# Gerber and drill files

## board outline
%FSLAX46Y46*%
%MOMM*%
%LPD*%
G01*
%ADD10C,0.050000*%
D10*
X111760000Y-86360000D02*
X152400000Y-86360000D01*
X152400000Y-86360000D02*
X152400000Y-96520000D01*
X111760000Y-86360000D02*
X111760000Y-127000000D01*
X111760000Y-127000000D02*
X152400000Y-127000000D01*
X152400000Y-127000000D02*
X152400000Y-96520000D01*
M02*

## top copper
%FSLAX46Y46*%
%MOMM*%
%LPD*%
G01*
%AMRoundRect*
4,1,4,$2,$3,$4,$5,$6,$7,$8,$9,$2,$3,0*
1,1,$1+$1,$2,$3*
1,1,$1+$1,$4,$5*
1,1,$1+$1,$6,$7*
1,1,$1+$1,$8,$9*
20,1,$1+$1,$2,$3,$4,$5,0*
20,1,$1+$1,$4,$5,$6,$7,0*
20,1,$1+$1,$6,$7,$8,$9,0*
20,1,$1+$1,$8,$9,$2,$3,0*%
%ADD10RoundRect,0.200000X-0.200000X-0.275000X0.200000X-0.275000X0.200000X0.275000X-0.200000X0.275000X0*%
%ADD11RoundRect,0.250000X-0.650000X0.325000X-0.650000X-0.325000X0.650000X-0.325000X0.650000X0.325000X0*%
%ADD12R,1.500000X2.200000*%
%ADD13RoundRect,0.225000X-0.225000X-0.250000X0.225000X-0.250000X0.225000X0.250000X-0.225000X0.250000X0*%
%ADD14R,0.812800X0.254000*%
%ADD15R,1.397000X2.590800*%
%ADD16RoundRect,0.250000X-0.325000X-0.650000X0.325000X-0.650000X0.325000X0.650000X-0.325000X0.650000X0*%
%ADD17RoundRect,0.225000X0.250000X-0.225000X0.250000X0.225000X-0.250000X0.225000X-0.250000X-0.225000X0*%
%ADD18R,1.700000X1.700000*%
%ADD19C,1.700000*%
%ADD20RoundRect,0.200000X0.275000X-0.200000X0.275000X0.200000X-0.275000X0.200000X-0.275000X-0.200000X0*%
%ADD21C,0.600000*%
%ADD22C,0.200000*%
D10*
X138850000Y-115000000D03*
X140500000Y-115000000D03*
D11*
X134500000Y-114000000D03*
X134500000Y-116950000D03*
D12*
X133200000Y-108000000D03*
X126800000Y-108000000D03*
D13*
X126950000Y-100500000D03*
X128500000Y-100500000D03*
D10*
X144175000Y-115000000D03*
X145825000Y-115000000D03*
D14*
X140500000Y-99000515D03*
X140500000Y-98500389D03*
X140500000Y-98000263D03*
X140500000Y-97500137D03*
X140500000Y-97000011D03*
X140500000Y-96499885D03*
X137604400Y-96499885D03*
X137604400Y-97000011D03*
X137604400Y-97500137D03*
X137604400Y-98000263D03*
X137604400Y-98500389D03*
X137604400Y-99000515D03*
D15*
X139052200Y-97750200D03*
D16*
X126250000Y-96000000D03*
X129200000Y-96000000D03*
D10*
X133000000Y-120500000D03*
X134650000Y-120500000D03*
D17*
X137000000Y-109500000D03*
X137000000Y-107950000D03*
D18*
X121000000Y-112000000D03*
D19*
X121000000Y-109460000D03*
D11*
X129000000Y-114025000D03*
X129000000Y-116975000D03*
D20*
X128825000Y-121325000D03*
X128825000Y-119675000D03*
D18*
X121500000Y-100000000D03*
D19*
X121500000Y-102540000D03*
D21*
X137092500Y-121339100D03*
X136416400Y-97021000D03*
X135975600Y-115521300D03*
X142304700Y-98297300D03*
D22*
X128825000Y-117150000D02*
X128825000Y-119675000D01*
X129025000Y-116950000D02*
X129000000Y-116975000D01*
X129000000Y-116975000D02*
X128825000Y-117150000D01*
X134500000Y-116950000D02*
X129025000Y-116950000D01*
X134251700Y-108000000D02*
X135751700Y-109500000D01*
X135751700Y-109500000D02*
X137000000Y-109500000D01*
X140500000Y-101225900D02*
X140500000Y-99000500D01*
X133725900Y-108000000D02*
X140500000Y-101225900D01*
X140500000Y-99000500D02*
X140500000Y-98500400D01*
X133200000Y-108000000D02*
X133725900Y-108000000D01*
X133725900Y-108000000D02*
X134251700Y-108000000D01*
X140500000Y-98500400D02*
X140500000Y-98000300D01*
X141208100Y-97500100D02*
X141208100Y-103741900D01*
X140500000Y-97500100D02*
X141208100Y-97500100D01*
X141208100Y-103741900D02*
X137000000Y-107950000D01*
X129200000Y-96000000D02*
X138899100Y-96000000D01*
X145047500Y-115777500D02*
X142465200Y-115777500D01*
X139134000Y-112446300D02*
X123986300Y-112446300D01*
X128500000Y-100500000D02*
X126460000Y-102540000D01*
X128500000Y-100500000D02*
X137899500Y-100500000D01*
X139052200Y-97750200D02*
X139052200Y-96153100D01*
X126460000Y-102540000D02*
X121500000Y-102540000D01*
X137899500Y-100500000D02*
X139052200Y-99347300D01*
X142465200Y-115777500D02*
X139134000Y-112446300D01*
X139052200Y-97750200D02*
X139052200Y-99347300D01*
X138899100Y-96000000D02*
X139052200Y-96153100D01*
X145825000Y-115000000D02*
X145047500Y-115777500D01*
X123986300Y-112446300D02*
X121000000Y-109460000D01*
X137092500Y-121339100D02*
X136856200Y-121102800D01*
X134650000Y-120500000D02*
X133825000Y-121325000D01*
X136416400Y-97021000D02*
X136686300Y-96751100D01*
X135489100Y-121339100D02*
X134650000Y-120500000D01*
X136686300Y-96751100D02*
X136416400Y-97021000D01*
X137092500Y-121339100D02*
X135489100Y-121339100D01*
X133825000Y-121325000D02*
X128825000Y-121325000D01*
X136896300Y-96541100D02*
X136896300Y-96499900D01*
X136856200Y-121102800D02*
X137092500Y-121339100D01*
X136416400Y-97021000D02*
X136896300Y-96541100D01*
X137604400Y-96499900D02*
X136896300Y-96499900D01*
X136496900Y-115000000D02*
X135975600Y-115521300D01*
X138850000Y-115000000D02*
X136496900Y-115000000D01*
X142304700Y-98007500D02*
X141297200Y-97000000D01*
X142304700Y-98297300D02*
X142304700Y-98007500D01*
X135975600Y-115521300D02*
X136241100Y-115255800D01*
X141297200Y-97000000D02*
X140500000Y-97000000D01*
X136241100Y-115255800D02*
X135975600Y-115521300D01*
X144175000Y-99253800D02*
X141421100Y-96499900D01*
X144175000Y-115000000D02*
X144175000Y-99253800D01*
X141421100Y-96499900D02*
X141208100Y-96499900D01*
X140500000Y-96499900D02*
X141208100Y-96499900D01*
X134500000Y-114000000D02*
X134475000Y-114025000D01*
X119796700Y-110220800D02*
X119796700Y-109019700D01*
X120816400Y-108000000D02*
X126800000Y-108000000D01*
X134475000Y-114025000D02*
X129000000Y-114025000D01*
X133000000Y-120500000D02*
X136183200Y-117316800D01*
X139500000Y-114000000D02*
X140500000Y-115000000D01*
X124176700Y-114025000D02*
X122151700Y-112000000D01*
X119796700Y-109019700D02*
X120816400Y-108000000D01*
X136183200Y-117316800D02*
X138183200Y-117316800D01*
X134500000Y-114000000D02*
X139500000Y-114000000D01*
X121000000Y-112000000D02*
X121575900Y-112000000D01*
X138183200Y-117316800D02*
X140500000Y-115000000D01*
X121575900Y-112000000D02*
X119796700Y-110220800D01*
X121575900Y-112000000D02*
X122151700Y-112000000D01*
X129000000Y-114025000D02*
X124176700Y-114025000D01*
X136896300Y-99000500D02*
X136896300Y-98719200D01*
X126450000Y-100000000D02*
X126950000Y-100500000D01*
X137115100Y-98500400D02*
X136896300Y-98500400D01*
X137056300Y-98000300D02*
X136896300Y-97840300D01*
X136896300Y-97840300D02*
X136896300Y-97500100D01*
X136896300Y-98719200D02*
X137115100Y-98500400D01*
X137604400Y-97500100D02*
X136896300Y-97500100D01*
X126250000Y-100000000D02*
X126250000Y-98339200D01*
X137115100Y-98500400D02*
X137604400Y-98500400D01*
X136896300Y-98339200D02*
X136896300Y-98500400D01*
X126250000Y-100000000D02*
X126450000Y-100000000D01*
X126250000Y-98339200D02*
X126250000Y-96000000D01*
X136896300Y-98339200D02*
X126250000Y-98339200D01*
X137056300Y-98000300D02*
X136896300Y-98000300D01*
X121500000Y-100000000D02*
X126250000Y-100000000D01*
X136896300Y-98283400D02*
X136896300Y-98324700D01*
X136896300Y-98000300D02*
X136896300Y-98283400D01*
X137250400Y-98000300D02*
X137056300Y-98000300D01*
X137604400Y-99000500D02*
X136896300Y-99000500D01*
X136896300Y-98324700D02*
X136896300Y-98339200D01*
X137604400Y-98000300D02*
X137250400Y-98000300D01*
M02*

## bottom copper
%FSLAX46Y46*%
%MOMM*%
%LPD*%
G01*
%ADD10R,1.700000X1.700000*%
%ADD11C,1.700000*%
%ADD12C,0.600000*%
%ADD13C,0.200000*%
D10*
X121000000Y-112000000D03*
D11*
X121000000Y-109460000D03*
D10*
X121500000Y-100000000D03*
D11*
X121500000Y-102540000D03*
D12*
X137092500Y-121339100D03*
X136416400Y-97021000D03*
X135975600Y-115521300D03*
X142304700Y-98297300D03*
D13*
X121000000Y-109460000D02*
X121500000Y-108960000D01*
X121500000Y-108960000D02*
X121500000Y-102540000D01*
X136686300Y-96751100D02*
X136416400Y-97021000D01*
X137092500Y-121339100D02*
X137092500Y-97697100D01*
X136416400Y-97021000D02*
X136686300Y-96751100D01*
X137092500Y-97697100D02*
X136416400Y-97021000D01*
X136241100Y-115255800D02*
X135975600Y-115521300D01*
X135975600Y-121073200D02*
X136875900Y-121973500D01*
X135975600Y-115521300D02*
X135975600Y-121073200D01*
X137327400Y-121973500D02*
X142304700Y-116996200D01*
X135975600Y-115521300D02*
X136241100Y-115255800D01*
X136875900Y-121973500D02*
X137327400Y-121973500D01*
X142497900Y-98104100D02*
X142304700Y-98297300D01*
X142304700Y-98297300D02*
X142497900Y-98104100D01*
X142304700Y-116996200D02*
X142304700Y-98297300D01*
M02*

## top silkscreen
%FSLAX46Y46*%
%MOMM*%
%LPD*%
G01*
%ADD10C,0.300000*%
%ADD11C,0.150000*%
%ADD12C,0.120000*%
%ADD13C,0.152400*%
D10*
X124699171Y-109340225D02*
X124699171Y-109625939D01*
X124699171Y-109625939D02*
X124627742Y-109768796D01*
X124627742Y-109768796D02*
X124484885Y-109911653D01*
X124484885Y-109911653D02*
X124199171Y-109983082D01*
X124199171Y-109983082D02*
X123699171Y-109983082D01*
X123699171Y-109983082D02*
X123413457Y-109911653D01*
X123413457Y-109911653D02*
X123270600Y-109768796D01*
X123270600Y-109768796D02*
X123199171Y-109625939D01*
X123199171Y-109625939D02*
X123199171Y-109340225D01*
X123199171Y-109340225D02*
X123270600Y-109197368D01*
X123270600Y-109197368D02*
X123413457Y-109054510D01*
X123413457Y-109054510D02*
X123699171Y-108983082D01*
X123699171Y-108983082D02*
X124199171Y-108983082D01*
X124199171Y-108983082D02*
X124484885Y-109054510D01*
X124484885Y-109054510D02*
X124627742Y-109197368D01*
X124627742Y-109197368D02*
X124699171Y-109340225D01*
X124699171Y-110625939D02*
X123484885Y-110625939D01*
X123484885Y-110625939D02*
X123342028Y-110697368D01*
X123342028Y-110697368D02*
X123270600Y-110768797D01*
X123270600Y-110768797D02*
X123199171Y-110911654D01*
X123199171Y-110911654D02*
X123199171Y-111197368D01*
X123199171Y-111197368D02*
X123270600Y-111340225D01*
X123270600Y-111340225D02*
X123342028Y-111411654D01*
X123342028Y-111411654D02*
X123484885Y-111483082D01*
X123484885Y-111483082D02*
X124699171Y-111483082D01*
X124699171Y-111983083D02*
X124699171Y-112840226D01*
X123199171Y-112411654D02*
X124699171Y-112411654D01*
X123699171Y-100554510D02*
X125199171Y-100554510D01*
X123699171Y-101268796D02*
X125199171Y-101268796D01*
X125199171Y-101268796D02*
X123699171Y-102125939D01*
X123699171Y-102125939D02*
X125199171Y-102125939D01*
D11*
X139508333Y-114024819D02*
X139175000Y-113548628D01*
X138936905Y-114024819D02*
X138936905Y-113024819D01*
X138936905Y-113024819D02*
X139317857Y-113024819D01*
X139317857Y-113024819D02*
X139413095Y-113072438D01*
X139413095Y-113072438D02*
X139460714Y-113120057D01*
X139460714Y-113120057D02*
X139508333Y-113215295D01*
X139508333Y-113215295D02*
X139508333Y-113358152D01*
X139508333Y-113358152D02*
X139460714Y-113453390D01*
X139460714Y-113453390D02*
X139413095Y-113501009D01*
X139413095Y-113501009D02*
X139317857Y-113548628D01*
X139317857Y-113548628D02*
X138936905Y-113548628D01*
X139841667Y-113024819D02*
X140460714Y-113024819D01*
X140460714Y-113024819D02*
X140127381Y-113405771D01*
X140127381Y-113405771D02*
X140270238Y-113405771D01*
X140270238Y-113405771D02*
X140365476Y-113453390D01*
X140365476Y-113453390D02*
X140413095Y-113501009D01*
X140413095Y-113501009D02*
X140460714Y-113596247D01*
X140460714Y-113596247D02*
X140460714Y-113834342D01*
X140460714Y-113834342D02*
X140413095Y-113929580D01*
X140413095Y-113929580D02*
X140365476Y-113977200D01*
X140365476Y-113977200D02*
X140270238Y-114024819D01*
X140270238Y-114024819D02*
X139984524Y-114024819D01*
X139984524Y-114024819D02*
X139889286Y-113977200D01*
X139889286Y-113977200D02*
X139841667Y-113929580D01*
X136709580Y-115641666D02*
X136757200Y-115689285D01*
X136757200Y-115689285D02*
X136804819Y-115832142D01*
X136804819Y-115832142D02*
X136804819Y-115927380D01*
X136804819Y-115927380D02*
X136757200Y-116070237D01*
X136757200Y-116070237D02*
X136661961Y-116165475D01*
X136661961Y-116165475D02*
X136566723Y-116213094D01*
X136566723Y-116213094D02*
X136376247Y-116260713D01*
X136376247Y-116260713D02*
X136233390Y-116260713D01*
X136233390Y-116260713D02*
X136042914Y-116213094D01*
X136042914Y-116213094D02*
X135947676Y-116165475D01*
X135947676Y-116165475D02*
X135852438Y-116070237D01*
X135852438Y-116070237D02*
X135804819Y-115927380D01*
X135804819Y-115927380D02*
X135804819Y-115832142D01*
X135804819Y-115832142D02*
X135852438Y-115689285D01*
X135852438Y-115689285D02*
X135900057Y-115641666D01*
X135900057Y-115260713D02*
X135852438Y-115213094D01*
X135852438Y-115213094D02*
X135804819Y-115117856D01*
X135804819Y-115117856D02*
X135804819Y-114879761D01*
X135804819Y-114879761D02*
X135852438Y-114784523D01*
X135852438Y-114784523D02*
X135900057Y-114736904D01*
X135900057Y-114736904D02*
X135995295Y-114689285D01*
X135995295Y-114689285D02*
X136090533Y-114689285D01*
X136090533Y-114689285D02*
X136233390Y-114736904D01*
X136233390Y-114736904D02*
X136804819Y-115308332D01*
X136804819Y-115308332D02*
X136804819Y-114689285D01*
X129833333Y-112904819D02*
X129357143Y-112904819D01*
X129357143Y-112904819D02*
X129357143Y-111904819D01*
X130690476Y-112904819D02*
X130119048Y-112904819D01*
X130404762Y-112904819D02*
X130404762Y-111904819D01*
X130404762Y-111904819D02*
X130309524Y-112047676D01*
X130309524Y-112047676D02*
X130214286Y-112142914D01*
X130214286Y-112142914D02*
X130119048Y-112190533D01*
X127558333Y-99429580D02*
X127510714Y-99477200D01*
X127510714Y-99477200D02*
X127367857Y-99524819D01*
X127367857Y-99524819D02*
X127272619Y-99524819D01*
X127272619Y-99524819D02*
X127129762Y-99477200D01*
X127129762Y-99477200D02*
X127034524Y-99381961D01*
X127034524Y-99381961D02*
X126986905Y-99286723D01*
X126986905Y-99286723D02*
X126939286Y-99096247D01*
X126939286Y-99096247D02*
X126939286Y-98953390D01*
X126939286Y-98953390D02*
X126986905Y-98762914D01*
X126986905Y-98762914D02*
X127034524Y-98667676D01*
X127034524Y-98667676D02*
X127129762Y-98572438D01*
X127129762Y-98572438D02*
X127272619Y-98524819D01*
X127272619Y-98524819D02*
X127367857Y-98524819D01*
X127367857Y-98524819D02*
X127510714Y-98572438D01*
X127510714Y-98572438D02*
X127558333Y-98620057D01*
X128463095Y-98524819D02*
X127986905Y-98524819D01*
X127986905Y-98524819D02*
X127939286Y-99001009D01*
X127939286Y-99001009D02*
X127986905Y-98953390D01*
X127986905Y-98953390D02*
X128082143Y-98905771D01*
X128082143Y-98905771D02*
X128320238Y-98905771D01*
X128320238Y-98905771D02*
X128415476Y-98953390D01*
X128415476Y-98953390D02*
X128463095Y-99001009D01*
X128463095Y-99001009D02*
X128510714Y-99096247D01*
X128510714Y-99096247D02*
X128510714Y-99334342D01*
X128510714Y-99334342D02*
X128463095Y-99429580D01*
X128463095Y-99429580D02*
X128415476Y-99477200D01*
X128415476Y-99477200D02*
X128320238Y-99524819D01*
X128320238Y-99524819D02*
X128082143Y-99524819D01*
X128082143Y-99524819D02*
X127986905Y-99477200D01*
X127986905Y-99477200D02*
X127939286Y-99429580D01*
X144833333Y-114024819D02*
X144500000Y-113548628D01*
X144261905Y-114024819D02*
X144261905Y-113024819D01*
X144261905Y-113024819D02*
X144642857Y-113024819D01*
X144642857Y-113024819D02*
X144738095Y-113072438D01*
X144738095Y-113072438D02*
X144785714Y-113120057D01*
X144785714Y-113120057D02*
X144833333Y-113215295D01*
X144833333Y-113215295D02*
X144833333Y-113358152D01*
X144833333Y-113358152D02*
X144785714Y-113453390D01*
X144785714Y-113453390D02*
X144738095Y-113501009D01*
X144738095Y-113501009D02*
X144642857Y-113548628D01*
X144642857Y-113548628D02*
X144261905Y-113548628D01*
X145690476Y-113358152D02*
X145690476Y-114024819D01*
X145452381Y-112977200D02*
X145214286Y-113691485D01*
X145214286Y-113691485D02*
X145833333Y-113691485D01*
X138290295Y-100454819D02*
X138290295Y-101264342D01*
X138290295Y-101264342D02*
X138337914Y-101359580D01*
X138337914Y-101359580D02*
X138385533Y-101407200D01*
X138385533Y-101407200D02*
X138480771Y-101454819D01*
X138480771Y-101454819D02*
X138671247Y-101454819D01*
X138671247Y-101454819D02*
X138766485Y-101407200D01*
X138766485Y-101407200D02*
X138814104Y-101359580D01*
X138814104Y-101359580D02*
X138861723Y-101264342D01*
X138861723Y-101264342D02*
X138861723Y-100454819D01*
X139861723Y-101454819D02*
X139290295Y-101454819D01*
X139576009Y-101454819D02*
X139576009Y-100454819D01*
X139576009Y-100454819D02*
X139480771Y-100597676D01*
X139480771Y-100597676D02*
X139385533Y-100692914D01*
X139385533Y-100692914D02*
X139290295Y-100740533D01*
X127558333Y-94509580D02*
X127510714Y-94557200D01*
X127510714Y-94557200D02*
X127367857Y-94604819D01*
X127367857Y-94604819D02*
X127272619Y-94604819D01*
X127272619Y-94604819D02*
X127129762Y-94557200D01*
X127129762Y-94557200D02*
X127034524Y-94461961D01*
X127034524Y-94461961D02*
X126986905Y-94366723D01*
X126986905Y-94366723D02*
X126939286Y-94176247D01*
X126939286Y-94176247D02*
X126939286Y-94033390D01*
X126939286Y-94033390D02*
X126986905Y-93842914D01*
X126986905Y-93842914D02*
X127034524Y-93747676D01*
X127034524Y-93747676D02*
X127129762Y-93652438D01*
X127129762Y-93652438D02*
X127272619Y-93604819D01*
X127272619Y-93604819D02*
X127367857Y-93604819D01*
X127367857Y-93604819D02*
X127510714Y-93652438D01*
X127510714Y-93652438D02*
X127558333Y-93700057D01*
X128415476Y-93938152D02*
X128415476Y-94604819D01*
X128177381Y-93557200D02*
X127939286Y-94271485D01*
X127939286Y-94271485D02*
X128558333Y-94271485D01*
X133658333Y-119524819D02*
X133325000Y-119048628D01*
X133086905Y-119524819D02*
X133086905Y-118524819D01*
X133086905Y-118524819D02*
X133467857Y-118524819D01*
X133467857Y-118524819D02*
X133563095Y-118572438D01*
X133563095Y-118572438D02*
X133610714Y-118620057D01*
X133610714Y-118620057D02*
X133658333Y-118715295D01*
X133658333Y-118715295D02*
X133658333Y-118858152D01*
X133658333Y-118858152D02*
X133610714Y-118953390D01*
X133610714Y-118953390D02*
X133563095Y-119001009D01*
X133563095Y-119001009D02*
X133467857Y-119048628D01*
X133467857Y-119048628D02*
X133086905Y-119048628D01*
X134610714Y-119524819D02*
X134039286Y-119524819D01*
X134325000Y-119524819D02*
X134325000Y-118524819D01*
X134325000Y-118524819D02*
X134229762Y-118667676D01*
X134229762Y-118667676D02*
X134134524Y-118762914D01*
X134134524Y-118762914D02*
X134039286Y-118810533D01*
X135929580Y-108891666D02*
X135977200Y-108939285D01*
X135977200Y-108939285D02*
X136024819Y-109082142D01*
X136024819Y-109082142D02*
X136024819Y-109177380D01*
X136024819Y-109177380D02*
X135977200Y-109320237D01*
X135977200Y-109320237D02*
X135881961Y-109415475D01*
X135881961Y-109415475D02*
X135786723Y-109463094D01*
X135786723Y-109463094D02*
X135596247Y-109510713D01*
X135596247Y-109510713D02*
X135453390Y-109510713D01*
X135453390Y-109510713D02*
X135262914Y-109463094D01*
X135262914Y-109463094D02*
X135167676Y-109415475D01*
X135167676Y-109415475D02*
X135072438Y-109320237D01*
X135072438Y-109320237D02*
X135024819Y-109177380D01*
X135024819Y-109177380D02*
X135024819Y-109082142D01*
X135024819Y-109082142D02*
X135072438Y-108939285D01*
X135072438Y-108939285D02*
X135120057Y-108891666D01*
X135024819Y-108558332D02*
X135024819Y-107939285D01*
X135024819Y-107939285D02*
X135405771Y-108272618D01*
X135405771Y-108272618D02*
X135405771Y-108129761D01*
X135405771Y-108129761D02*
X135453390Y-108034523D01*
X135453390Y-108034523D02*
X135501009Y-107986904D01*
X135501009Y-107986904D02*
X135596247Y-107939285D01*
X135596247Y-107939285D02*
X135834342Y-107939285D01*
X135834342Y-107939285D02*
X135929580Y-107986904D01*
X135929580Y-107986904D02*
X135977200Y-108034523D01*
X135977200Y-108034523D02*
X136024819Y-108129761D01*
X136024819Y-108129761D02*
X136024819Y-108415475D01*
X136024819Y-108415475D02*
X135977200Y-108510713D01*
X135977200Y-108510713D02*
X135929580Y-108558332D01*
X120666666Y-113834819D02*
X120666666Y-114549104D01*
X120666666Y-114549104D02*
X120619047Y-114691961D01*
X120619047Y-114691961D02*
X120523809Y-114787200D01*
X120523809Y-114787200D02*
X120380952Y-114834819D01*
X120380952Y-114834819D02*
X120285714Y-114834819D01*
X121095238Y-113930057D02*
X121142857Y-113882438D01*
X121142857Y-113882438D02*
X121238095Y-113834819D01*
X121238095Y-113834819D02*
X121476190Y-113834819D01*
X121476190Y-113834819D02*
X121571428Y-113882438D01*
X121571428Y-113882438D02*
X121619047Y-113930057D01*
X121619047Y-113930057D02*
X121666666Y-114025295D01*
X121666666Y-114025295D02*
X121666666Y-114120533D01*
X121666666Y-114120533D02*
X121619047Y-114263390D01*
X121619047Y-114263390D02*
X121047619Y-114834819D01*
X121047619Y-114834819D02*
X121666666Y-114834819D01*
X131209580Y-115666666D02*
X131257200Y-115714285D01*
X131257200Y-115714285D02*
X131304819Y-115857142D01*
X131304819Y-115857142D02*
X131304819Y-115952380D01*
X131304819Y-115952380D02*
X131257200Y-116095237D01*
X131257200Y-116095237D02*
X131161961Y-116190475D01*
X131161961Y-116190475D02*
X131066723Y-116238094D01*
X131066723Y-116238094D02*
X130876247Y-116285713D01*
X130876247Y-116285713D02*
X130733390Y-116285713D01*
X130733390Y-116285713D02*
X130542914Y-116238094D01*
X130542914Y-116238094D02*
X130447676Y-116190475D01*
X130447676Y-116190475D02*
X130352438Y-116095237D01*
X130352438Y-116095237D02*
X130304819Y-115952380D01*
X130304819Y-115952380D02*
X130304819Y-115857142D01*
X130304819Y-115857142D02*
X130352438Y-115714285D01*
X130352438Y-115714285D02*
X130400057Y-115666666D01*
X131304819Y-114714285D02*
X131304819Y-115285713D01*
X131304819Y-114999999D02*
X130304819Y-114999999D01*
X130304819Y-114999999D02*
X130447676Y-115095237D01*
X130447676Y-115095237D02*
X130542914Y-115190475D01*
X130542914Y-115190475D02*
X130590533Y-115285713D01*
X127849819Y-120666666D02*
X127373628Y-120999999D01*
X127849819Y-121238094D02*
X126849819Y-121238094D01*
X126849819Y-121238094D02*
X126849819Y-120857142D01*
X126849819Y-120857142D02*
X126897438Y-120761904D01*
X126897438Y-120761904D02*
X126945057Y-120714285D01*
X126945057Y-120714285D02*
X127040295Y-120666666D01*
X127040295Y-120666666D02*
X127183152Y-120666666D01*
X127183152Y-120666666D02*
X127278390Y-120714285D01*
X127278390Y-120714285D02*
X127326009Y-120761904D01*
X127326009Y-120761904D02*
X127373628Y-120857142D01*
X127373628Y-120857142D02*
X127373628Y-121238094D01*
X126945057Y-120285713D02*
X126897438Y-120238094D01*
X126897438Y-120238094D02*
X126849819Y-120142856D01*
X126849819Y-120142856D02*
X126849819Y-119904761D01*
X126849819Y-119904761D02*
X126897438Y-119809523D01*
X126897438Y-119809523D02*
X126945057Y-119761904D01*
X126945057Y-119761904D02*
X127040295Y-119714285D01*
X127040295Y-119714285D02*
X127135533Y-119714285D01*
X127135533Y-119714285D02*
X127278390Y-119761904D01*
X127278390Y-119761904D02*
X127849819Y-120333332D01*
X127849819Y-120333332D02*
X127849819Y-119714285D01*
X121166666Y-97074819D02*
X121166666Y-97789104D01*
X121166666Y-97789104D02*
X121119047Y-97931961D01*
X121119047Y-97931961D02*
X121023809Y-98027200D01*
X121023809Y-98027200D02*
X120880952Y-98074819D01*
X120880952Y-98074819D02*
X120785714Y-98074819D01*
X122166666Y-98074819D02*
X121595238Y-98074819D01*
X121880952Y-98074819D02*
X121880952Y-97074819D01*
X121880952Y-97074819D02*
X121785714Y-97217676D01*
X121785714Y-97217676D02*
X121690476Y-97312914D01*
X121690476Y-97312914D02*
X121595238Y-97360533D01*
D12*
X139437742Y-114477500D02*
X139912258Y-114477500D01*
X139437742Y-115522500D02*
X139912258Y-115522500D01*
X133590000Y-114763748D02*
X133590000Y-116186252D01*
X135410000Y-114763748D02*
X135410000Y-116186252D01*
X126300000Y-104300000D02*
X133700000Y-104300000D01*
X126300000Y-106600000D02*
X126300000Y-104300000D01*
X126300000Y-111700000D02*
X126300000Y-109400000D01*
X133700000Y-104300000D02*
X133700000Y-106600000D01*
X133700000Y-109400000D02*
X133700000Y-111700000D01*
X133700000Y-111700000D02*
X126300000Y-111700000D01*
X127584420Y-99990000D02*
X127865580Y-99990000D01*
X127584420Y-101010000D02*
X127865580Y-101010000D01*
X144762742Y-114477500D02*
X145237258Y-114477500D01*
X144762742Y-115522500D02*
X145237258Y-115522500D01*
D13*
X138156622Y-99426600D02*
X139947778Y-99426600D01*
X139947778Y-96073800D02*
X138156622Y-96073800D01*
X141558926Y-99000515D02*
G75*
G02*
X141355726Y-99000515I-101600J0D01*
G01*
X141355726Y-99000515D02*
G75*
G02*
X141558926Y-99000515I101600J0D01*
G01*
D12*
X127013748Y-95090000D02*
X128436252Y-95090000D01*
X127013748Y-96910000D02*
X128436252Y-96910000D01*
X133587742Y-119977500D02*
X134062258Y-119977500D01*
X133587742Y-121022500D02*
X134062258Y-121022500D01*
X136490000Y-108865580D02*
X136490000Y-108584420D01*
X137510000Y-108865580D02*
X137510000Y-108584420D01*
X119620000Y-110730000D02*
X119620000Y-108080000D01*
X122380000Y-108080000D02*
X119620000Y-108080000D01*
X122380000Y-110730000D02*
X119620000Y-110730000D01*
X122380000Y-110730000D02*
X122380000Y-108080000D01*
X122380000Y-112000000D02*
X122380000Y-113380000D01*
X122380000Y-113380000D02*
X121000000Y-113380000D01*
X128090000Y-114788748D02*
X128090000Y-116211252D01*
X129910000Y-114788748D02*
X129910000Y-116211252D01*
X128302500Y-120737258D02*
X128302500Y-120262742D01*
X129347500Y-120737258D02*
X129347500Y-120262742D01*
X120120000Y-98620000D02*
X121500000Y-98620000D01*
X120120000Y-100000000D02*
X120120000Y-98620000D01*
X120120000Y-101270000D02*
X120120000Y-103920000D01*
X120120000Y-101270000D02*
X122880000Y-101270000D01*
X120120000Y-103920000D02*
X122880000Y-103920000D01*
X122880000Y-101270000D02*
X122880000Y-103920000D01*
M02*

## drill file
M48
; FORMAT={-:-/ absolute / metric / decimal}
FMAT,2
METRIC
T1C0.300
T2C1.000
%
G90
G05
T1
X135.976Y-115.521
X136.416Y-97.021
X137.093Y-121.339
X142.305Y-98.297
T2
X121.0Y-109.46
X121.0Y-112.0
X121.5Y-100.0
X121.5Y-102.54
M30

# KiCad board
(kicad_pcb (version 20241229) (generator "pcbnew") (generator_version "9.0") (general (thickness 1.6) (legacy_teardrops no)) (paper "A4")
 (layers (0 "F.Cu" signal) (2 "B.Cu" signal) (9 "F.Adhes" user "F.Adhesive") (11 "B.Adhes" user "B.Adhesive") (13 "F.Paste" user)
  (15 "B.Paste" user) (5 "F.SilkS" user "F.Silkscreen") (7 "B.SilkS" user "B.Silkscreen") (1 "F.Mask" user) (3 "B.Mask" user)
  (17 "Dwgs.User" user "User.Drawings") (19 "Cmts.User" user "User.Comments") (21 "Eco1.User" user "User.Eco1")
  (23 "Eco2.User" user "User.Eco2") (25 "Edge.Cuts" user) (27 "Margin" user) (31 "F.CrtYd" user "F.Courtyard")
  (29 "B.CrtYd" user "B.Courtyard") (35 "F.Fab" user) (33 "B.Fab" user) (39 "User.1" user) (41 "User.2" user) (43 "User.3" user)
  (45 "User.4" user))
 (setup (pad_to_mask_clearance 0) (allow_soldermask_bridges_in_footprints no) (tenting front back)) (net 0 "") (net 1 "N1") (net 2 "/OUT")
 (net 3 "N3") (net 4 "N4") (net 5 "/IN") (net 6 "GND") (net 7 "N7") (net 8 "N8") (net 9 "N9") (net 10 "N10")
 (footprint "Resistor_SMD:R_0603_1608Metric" (layer "F.Cu") (at 139.675 115)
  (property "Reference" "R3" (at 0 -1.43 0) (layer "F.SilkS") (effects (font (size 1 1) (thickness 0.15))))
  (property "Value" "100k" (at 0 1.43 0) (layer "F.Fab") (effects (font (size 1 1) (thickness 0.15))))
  (fp_line (start -0.237258 -0.5225) (end 0.237258 -0.5225) (stroke (width 0.12) (type solid)) (layer "F.SilkS"))
  (fp_line (start -0.237258 0.5225) (end 0.237258 0.5225) (stroke (width 0.12) (type solid)) (layer "F.SilkS"))
  (pad "1" smd roundrect (at -0.825 0) (size 0.8 0.95) (layers "F.Cu" "F.Mask" "F.Paste") (roundrect_rratio 0.25) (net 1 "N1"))
  (pad "2" smd roundrect (at 0.825 0) (size 0.8 0.95) (layers "F.Cu" "F.Mask" "F.Paste") (roundrect_rratio 0.25) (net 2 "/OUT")))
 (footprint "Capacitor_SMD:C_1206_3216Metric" (layer "F.Cu") (at 134.5 115.475 -90)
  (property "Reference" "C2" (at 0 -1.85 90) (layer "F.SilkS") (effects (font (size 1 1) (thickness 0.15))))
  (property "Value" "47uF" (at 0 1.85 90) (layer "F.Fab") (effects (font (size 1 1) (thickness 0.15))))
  (fp_line (start -0.711252 0.91) (end 0.711252 0.91) (stroke (width 0.12) (type solid)) (layer "F.SilkS"))
  (fp_line (start -0.711252 -0.91) (end 0.711252 -0.91) (stroke (width 0.12) (type solid)) (layer "F.SilkS"))
  (pad "1" smd roundrect (at -1.475 0 270) (size 1.15 1.8) (layers "F.Cu" "F.Mask" "F.Paste") (roundrect_rratio 0.217391) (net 2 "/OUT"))
  (pad "2" smd roundrect (at 1.475 0 270) (size 1.15 1.8) (layers "F.Cu" "F.Mask" "F.Paste") (roundrect_rratio 0.217391) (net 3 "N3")))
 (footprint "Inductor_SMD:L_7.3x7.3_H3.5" (layer "F.Cu") (at 130 108 180)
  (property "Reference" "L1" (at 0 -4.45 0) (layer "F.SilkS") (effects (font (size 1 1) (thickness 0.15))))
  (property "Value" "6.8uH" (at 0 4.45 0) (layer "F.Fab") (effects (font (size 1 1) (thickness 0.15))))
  (fp_line (start 3.7 3.7) (end -3.7 3.7) (stroke (width 0.12) (type solid)) (layer "F.SilkS"))
  (fp_line (start 3.7 1.4) (end 3.7 3.7) (stroke (width 0.12) (type solid)) (layer "F.SilkS"))
  (fp_line (start 3.7 -3.7) (end 3.7 -1.4) (stroke (width 0.12) (type solid)) (layer "F.SilkS"))
  (fp_line (start -3.7 3.7) (end -3.7 1.4) (stroke (width 0.12) (type solid)) (layer "F.SilkS"))
  (fp_line (start -3.7 -1.4) (end -3.7 -3.7) (stroke (width 0.12) (type solid)) (layer "F.SilkS"))
  (fp_line (start -3.7 -3.7) (end 3.7 -3.7) (stroke (width 0.12) (type solid)) (layer "F.SilkS"))
  (pad "1" smd rect (at -3.2 0 180) (size 1.5 2.2) (layers "F.Cu" "F.Mask" "F.Paste") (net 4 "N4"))
  (pad "2" smd rect (at 3.2 0 180) (size 1.5 2.2) (layers "F.Cu" "F.Mask" "F.Paste") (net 2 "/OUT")))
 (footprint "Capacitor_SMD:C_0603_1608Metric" (layer "F.Cu") (at 127.725 100.5)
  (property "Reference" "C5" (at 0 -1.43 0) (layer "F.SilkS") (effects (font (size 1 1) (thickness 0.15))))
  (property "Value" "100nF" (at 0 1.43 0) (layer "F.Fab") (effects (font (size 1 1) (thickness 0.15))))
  (fp_line (start -0.14058 -0.51) (end 0.14058 -0.51) (stroke (width 0.12) (type solid)) (layer "F.SilkS"))
  (fp_line (start -0.14058 0.51) (end 0.14058 0.51) (stroke (width 0.12) (type solid)) (layer "F.SilkS"))
  (pad "1" smd roundrect (at -0.775 0) (size 0.9 0.95) (layers "F.Cu" "F.Mask" "F.Paste") (roundrect_rratio 0.25) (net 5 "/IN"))
  (pad "2" smd roundrect (at 0.775 0) (size 0.9 0.95) (layers "F.Cu" "F.Mask" "F.Paste") (roundrect_rratio 0.25) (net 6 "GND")))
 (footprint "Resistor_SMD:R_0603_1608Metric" (layer "F.Cu") (at 145 115)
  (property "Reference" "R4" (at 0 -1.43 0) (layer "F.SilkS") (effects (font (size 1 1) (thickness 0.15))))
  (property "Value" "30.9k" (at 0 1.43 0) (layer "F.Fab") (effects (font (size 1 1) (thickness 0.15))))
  (fp_line (start -0.237258 -0.5225) (end 0.237258 -0.5225) (stroke (width 0.12) (type solid)) (layer "F.SilkS"))
  (fp_line (start -0.237258 0.5225) (end 0.237258 0.5225) (stroke (width 0.12) (type solid)) (layer "F.SilkS"))
  (pad "1" smd roundrect (at -0.825 0) (size 0.8 0.95) (layers "F.Cu" "F.Mask" "F.Paste") (roundrect_rratio 0.25) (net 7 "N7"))
  (pad "2" smd roundrect (at 0.825 0) (size 0.8 0.95) (layers "F.Cu" "F.Mask" "F.Paste") (roundrect_rratio 0.25) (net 6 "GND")))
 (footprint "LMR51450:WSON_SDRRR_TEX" (layer "F.Cu") (at 139.0522 97.7502 180)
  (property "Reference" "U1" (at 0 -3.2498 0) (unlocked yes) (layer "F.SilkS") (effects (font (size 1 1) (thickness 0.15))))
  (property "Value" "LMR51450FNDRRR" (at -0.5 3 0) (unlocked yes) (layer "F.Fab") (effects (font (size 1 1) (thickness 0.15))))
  (fp_line (start 0.895578 -1.6764) (end -0.895578 -1.6764) (stroke (width 0.1524) (type solid)) (layer "F.SilkS"))
  (fp_line (start -0.895578 1.6764) (end 0.895578 1.6764) (stroke (width 0.1524) (type solid)) (layer "F.SilkS"))
  (fp_circle (center -2.405126 -1.250315) (end -2.303526 -1.250315) (stroke (width 0.1524) (type solid)) (fill no) (layer "F.SilkS"))
  (pad "1" smd rect (at -1.4478 -1.250315 180) (size 0.8128 0.254) (layers "F.Cu" "F.Mask" "F.Paste") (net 4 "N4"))
  (pad "2" smd rect (at -1.4478 -0.750189 180) (size 0.8128 0.254) (layers "F.Cu" "F.Mask" "F.Paste") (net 4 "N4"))
  (pad "3" smd rect (at -1.4478 -0.250063 180) (size 0.8128 0.254) (layers "F.Cu" "F.Mask" "F.Paste") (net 4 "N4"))
  (pad "4" smd rect (at -1.4478 0.250063 180) (size 0.8128 0.254) (layers "F.Cu" "F.Mask" "F.Paste") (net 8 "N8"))
  (pad "5" smd rect (at -1.4478 0.750189 180) (size 0.8128 0.254) (layers "F.Cu" "F.Mask" "F.Paste") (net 1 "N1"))
  (pad "6" smd rect (at -1.4478 1.250315 180) (size 0.8128 0.254) (layers "F.Cu" "F.Mask" "F.Paste") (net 7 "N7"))
  (pad "7" smd rect (at 1.4478 1.250315 180) (size 0.8128 0.254) (layers "F.Cu" "F.Mask" "F.Paste") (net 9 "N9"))
  (pad "8" smd rect (at 1.4478 0.750189 180) (size 0.8128 0.254) (layers "F.Cu" "F.Mask" "F.Paste") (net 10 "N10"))
  (pad "9" smd rect (at 1.4478 0.250063 180) (size 0.8128 0.254) (layers "F.Cu" "F.Mask" "F.Paste") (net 5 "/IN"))
  (pad "10" smd rect (at 1.4478 -0.250063 180) (size 0.8128 0.254) (layers "F.Cu" "F.Mask" "F.Paste") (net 5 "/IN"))
  (pad "11" smd rect (at 1.4478 -0.750189 180) (size 0.8128 0.254) (layers "F.Cu" "F.Mask" "F.Paste") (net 5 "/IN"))
  (pad "12" smd rect (at 1.4478 -1.250315 180) (size 0.8128 0.254) (layers "F.Cu" "F.Mask" "F.Paste") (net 5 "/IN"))
  (pad "13" smd rect (at 0 0 180) (size 1.397 2.5908) (layers "F.Cu" "F.Mask" "F.Paste") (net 6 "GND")))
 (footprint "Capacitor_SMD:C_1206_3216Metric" (layer "F.Cu") (at 127.725 96)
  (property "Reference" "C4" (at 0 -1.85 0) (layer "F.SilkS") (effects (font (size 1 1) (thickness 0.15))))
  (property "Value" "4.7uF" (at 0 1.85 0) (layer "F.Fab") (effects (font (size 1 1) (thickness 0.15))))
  (fp_line (start -0.711252 -0.91) (end 0.711252 -0.91) (stroke (width 0.12) (type solid)) (layer "F.SilkS"))
  (fp_line (start -0.711252 0.91) (end 0.711252 0.91) (stroke (width 0.12) (type solid)) (layer "F.SilkS"))
  (pad "1" smd roundrect (at -1.475 0) (size 1.15 1.8) (layers "F.Cu" "F.Mask" "F.Paste") (roundrect_rratio 0.217391) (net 5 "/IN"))
  (pad "2" smd roundrect (at 1.475 0) (size 1.15 1.8) (layers "F.Cu" "F.Mask" "F.Paste") (roundrect_rratio 0.217391) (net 6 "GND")))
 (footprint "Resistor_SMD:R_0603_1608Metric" (layer "F.Cu") (at 133.825 120.5)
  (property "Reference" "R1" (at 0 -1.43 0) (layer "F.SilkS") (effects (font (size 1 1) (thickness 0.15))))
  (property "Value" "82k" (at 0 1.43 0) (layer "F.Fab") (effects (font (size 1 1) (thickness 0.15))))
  (fp_line (start -0.237258 -0.5225) (end 0.237258 -0.5225) (stroke (width 0.12) (type solid)) (layer "F.SilkS"))
  (fp_line (start -0.237258 0.5225) (end 0.237258 0.5225) (stroke (width 0.12) (type solid)) (layer "F.SilkS"))
  (pad "1" smd roundrect (at -0.825 0) (size 0.8 0.95) (layers "F.Cu" "F.Mask" "F.Paste") (roundrect_rratio 0.25) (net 2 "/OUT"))
  (pad "2" smd roundrect (at 0.825 0) (size 0.8 0.95) (layers "F.Cu" "F.Mask" "F.Paste") (roundrect_rratio 0.25) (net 9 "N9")))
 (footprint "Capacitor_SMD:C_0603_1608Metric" (layer "F.Cu") (at 137 108.725 90)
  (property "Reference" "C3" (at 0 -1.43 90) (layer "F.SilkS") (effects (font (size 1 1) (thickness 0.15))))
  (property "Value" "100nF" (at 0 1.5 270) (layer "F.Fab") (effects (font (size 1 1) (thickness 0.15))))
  (fp_line (start -0.14058 -0.51) (end 0.14058 -0.51) (stroke (width 0.12) (type solid)) (layer "F.SilkS"))
  (fp_line (start -0.14058 0.51) (end 0.14058 0.51) (stroke (width 0.12) (type solid)) (layer "F.SilkS"))
  (pad "1" smd roundrect (at -0.775 0 90) (size 0.9 0.95) (layers "F.Cu" "F.Mask" "F.Paste") (roundrect_rratio 0.25) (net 4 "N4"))
  (pad "2" smd roundrect (at 0.775 0 90) (size 0.9 0.95) (layers "F.Cu" "F.Mask" "F.Paste") (roundrect_rratio 0.25) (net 8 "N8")))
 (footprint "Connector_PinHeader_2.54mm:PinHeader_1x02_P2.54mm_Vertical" (layer "F.Cu") (at 121 112 180)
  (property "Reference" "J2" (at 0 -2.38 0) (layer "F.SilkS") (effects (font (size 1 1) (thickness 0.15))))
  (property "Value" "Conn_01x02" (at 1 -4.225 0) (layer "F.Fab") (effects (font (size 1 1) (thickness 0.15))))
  (fp_line (start 1.38 1.27) (end 1.38 3.92) (stroke (width 0.12) (type solid)) (layer "F.SilkS"))
  (fp_line (start -1.38 3.92) (end 1.38 3.92) (stroke (width 0.12) (type solid)) (layer "F.SilkS"))
  (fp_line (start -1.38 1.27) (end 1.38 1.27) (stroke (width 0.12) (type solid)) (layer "F.SilkS"))
  (fp_line (start -1.38 1.27) (end -1.38 3.92) (stroke (width 0.12) (type solid)) (layer "F.SilkS"))
  (fp_line (start -1.38 0) (end -1.38 -1.38) (stroke (width 0.12) (type solid)) (layer "F.SilkS"))
  (fp_line (start -1.38 -1.38) (end 0 -1.38) (stroke (width 0.12) (type solid)) (layer "F.SilkS"))
  (pad "1" thru_hole rect (at 0 0 180) (size 1.7 1.7) (drill 1) (layers "*.Cu" "*.Mask") (remove_unused_layers no) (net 2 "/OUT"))
  (pad "2" thru_hole circle (at 0 2.54 180) (size 1.7 1.7) (drill 1) (layers "*.Cu" "*.Mask") (remove_unused_layers no) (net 6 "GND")))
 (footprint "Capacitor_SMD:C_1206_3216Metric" (layer "F.Cu") (at 129 115.5 -90)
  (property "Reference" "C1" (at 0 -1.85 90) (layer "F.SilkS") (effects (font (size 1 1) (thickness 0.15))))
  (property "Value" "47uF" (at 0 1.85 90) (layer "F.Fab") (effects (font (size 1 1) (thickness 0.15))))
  (fp_line (start -0.711252 0.91) (end 0.711252 0.91) (stroke (width 0.12) (type solid)) (layer "F.SilkS"))
  (fp_line (start -0.711252 -0.91) (end 0.711252 -0.91) (stroke (width 0.12) (type solid)) (layer "F.SilkS"))
  (pad "1" smd roundrect (at -1.475 0 270) (size 1.15 1.8) (layers "F.Cu" "F.Mask" "F.Paste") (roundrect_rratio 0.217391) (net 2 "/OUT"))
  (pad "2" smd roundrect (at 1.475 0 270) (size 1.15 1.8) (layers "F.Cu" "F.Mask" "F.Paste") (roundrect_rratio 0.217391) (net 3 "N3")))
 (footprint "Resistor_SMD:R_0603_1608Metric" (layer "F.Cu") (at 128.825 120.5 90)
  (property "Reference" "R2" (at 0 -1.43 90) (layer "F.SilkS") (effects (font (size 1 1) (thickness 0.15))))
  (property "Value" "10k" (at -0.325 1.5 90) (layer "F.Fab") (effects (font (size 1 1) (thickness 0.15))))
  (fp_line (start -0.237258 -0.5225) (end 0.237258 -0.5225) (stroke (width 0.12) (type solid)) (layer "F.SilkS"))
  (fp_line (start -0.237258 0.5225) (end 0.237258 0.5225) (stroke (width 0.12) (type solid)) (layer "F.SilkS"))
  (pad "1" smd roundrect (at -0.825 0 90) (size 0.8 0.95) (layers "F.Cu" "F.Mask" "F.Paste") (roundrect_rratio 0.25) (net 9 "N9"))
  (pad "2" smd roundrect (at 0.825 0 90) (size 0.8 0.95) (layers "F.Cu" "F.Mask" "F.Paste") (roundrect_rratio 0.25) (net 3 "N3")))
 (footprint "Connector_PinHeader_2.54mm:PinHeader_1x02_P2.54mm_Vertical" (layer "F.Cu") (at 121.5 100)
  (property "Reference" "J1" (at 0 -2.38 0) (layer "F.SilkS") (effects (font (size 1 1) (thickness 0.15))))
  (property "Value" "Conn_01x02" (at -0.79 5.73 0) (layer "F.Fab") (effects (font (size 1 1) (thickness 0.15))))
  (fp_line (start -1.38 -1.38) (end 0 -1.38) (stroke (width 0.12) (type solid)) (layer "F.SilkS"))
  (fp_line (start -1.38 0) (end -1.38 -1.38) (stroke (width 0.12) (type solid)) (layer "F.SilkS"))
  (fp_line (start -1.38 1.27) (end -1.38 3.92) (stroke (width 0.12) (type solid)) (layer "F.SilkS"))
  (fp_line (start -1.38 1.27) (end 1.38 1.27) (stroke (width 0.12) (type solid)) (layer "F.SilkS"))
  (fp_line (start -1.38 3.92) (end 1.38 3.92) (stroke (width 0.12) (type solid)) (layer "F.SilkS"))
  (fp_line (start 1.38 1.27) (end 1.38 3.92) (stroke (width 0.12) (type solid)) (layer "F.SilkS"))
  (pad "1" thru_hole rect (at 0 0) (size 1.7 1.7) (drill 1) (layers "*.Cu" "*.Mask") (remove_unused_layers no) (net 5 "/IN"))
  (pad "2" thru_hole circle (at 0 2.54) (size 1.7 1.7) (drill 1) (layers "*.Cu" "*.Mask") (remove_unused_layers no) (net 6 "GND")))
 (gr_line (start 111.76 86.36) (end 152.4 86.36) (stroke (width 0.05) (type default)) (layer "Edge.Cuts"))
 (gr_line (start 152.4 86.36) (end 152.4 96.52) (stroke (width 0.05) (type default)) (layer "Edge.Cuts"))
 (gr_line (start 111.76 86.36) (end 111.76 127) (stroke (width 0.05) (type default)) (layer "Edge.Cuts"))
 (gr_line (start 111.76 127) (end 152.4 127) (stroke (width 0.05) (type default)) (layer "Edge.Cuts"))
 (gr_line (start 152.4 127) (end 152.4 96.52) (stroke (width 0.05) (type default)) (layer "Edge.Cuts"))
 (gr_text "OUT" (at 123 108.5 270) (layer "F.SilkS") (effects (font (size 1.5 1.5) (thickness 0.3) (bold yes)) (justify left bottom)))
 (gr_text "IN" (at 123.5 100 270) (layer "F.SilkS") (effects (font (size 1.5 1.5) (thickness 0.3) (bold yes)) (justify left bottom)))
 (segment (start 128.825 117.15) (end 128.825 119.675) (width 0.2) (layer "F.Cu") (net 3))
 (segment (start 129.025 116.95) (end 129 116.975) (width 0.2) (layer "F.Cu") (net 3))
 (segment (start 129 116.975) (end 128.825 117.15) (width 0.2) (layer "F.Cu") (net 3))
 (segment (start 134.5 116.95) (end 129.025 116.95) (width 0.2) (layer "F.Cu") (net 3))
 (segment (start 134.2517 108) (end 135.7517 109.5) (width 0.2) (layer "F.Cu") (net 4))
 (segment (start 135.7517 109.5) (end 137 109.5) (width 0.2) (layer "F.Cu") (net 4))
 (segment (start 140.5 101.2259) (end 140.5 99.0005) (width 0.2) (layer "F.Cu") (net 4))
 (segment (start 133.7259 108) (end 140.5 101.2259) (width 0.2) (layer "F.Cu") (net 4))
 (segment (start 140.5 99.0005) (end 140.5 98.5004) (width 0.2) (layer "F.Cu") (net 4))
 (segment (start 133.2 108) (end 133.7259 108) (width 0.2) (layer "F.Cu") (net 4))
 (segment (start 133.7259 108) (end 134.2517 108) (width 0.2) (layer "F.Cu") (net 4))
 (segment (start 140.5 98.5004) (end 140.5 98.0003) (width 0.2) (layer "F.Cu") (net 4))
 (segment (start 141.2081 97.5001) (end 141.2081 103.7419) (width 0.2) (layer "F.Cu") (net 8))
 (segment (start 140.5 97.5001) (end 141.2081 97.5001) (width 0.2) (layer "F.Cu") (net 8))
 (segment (start 141.2081 103.7419) (end 137 107.95) (width 0.2) (layer "F.Cu") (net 8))
 (segment (start 129.2 96) (end 138.8991 96) (width 0.2) (layer "F.Cu") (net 6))
 (segment (start 145.0475 115.7775) (end 142.4652 115.7775) (width 0.2) (layer "F.Cu") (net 6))
 (segment (start 139.134 112.4463) (end 123.9863 112.4463) (width 0.2) (layer "F.Cu") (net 6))
 (segment (start 128.5 100.5) (end 126.46 102.54) (width 0.2) (layer "F.Cu") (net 6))
 (segment (start 128.5 100.5) (end 137.8995 100.5) (width 0.2) (layer "F.Cu") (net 6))
 (segment (start 139.0522 97.7502) (end 139.0522 96.1531) (width 0.2) (layer "F.Cu") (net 6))
 (segment (start 126.46 102.54) (end 121.5 102.54) (width 0.2) (layer "F.Cu") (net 6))
 (segment (start 137.8995 100.5) (end 139.0522 99.3473) (width 0.2) (layer "F.Cu") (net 6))
 (segment (start 142.4652 115.7775) (end 139.134 112.4463) (width 0.2) (layer "F.Cu") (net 6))
 (segment (start 139.0522 97.7502) (end 139.0522 99.3473) (width 0.2) (layer "F.Cu") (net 6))
 (segment (start 138.8991 96) (end 139.0522 96.1531) (width 0.2) (layer "F.Cu") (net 6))
 (segment (start 145.825 115) (end 145.0475 115.7775) (width 0.2) (layer "F.Cu") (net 6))
 (segment (start 123.9863 112.4463) (end 121 109.46) (width 0.2) (layer "F.Cu") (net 6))
 (segment (start 121 109.46) (end 121.5 108.96) (width 0.2) (layer "B.Cu") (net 6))
 (segment (start 121.5 108.96) (end 121.5 102.54) (width 0.2) (layer "B.Cu") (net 6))
 (segment (start 137.0925 121.3391) (end 136.8562 121.1028) (width 0.2) (layer "F.Cu") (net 9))
 (segment (start 134.65 120.5) (end 133.825 121.325) (width 0.2) (layer "F.Cu") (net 9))
 (segment (start 136.4164 97.021) (end 136.6863 96.7511) (width 0.2) (layer "F.Cu") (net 9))
 (segment (start 135.4891 121.3391) (end 134.65 120.5) (width 0.2) (layer "F.Cu") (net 9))
 (segment (start 136.6863 96.7511) (end 136.4164 97.021) (width 0.2) (layer "F.Cu") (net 9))
 (segment (start 137.0925 121.3391) (end 135.4891 121.3391) (width 0.2) (layer "F.Cu") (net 9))
 (segment (start 133.825 121.325) (end 128.825 121.325) (width 0.2) (layer "F.Cu") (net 9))
 (segment (start 136.8963 96.5411) (end 136.8963 96.4999) (width 0.2) (layer "F.Cu") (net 9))
 (segment (start 136.8562 121.1028) (end 137.0925 121.3391) (width 0.2) (layer "F.Cu") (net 9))
 (segment (start 136.4164 97.021) (end 136.8963 96.5411) (width 0.2) (layer "F.Cu") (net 9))
 (segment (start 137.6044 96.4999) (end 136.8963 96.4999) (width 0.2) (layer "F.Cu") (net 9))
 (via (at 137.0925 121.3391) (size 0.6) (drill 0.3) (layers "F.Cu" "B.Cu") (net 9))
 (via (at 136.4164 97.021) (size 0.6) (drill 0.3) (layers "F.Cu" "B.Cu") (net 9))
 (segment (start 136.6863 96.7511) (end 136.4164 97.021) (width 0.2) (layer "B.Cu") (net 9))
 (segment (start 137.0925 121.3391) (end 137.0925 97.6971) (width 0.2) (layer "B.Cu") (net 9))
 (segment (start 136.4164 97.021) (end 136.6863 96.7511) (width 0.2) (layer "B.Cu") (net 9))
 (segment (start 137.0925 97.6971) (end 136.4164 97.021) (width 0.2) (layer "B.Cu") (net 9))
 (segment (start 136.4969 115) (end 135.9756 115.5213) (width 0.2) (layer "F.Cu") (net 1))
 (segment (start 138.85 115) (end 136.4969 115) (width 0.2) (layer "F.Cu") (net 1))
 (segment (start 142.3047 98.0075) (end 141.2972 97) (width 0.2) (layer "F.Cu") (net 1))
 (segment (start 142.3047 98.2973) (end 142.3047 98.0075) (width 0.2) (layer "F.Cu") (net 1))
 (segment (start 135.9756 115.5213) (end 136.2411 115.2558) (width 0.2) (layer "F.Cu") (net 1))
 (segment (start 141.2972 97) (end 140.5 97) (width 0.2) (layer "F.Cu") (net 1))
 (segment (start 136.2411 115.2558) (end 135.9756 115.5213) (width 0.2) (layer "F.Cu") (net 1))
 (via (at 135.9756 115.5213) (size 0.6) (drill 0.3) (layers "F.Cu" "B.Cu") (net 1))
 (via (at 142.3047 98.2973) (size 0.6) (drill 0.3) (layers "F.Cu" "B.Cu") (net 1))
 (segment (start 136.2411 115.2558) (end 135.9756 115.5213) (width 0.2) (layer "B.Cu") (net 1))
 (segment (start 135.9756 121.0732) (end 136.8759 121.9735) (width 0.2) (layer "B.Cu") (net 1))
 (segment (start 135.9756 115.5213) (end 135.9756 121.0732) (width 0.2) (layer "B.Cu") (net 1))
 (segment (start 137.3274 121.9735) (end 142.3047 116.9962) (width 0.2) (layer "B.Cu") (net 1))
 (segment (start 135.9756 115.5213) (end 136.2411 115.2558) (width 0.2) (layer "B.Cu") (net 1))
 (segment (start 136.8759 121.9735) (end 137.3274 121.9735) (width 0.2) (layer "B.Cu") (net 1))
 (segment (start 142.4979 98.1041) (end 142.3047 98.2973) (width 0.2) (layer "B.Cu") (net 1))
 (segment (start 142.3047 98.2973) (end 142.4979 98.1041) (width 0.2) (layer "B.Cu") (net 1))
 (segment (start 142.3047 116.9962) (end 142.3047 98.2973) (width 0.2) (layer "B.Cu") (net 1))
 (segment (start 144.175 99.2538) (end 141.4211 96.4999) (width 0.2) (layer "F.Cu") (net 7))
 (segment (start 144.175 115) (end 144.175 99.2538) (width 0.2) (layer "F.Cu") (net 7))
 (segment (start 141.4211 96.4999) (end 141.2081 96.4999) (width 0.2) (layer "F.Cu") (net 7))
 (segment (start 140.5 96.4999) (end 141.2081 96.4999) (width 0.2) (layer "F.Cu") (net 7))
 (segment (start 134.5 114) (end 134.475 114.025) (width 0.2) (layer "F.Cu") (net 2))
 (segment (start 119.7967 110.2208) (end 119.7967 109.0197) (width 0.2) (layer "F.Cu") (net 2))
 (segment (start 120.8164 108) (end 126.8 108) (width 0.2) (layer "F.Cu") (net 2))
 (segment (start 134.475 114.025) (end 129 114.025) (width 0.2) (layer "F.Cu") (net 2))
 (segment (start 133 120.5) (end 136.1832 117.3168) (width 0.2) (layer "F.Cu") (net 2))
 (segment (start 139.5 114) (end 140.5 115) (width 0.2) (layer "F.Cu") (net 2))
 (segment (start 124.1767 114.025) (end 122.1517 112) (width 0.2) (layer "F.Cu") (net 2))
 (segment (start 119.7967 109.0197) (end 120.8164 108) (width 0.2) (layer "F.Cu") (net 2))
 (segment (start 136.1832 117.3168) (end 138.1832 117.3168) (width 0.2) (layer "F.Cu") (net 2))
 (segment (start 134.5 114) (end 139.5 114) (width 0.2) (layer "F.Cu") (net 2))
 (segment (start 121 112) (end 121.5759 112) (width 0.2) (layer "F.Cu") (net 2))
 (segment (start 138.1832 117.3168) (end 140.5 115) (width 0.2) (layer "F.Cu") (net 2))
 (segment (start 121.5759 112) (end 119.7967 110.2208) (width 0.2) (layer "F.Cu") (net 2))
 (segment (start 121.5759 112) (end 122.1517 112) (width 0.2) (layer "F.Cu") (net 2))
 (segment (start 129 114.025) (end 124.1767 114.025) (width 0.2) (layer "F.Cu") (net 2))
 (segment (start 136.8963 99.0005) (end 136.8963 98.7192) (width 0.2) (layer "F.Cu") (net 5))
 (segment (start 126.45 100) (end 126.95 100.5) (width 0.2) (layer "F.Cu") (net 5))
 (segment (start 137.1151 98.5004) (end 136.8963 98.5004) (width 0.2) (layer "F.Cu") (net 5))
 (segment (start 137.0563 98.0003) (end 136.8963 97.8403) (width 0.2) (layer "F.Cu") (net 5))
 (segment (start 136.8963 97.8403) (end 136.8963 97.5001) (width 0.2) (layer "F.Cu") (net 5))
 (segment (start 136.8963 98.7192) (end 137.1151 98.5004) (width 0.2) (layer "F.Cu") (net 5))
 (segment (start 137.6044 97.5001) (end 136.8963 97.5001) (width 0.2) (layer "F.Cu") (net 5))
 (segment (start 126.25 100) (end 126.25 98.3392) (width 0.2) (layer "F.Cu") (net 5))
 (segment (start 137.1151 98.5004) (end 137.6044 98.5004) (width 0.2) (layer "F.Cu") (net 5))
 (segment (start 136.8963 98.3392) (end 136.8963 98.5004) (width 0.2) (layer "F.Cu") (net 5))
 (segment (start 126.25 100) (end 126.45 100) (width 0.2) (layer "F.Cu") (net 5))
 (segment (start 126.25 98.3392) (end 126.25 96) (width 0.2) (layer "F.Cu") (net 5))
 (segment (start 136.8963 98.3392) (end 126.25 98.3392) (width 0.2) (layer "F.Cu") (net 5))
 (segment (start 137.0563 98.0003) (end 136.8963 98.0003) (width 0.2) (layer "F.Cu") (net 5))
 (segment (start 121.5 100) (end 126.25 100) (width 0.2) (layer "F.Cu") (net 5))
 (segment (start 136.8963 98.2834) (end 136.8963 98.3247) (width 0.2) (layer "F.Cu") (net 5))
 (segment (start 136.8963 98.0003) (end 136.8963 98.2834) (width 0.2) (layer "F.Cu") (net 5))
 (segment (start 137.2504 98.0003) (end 137.0563 98.0003) (width 0.2) (layer "F.Cu") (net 5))
 (segment (start 137.6044 99.0005) (end 136.8963 99.0005) (width 0.2) (layer "F.Cu") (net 5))
 (segment (start 136.8963 98.3247) (end 136.8963 98.3392) (width 0.2) (layer "F.Cu") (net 5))
 (segment (start 137.6044 98.0003) (end 137.2504 98.0003) (width 0.2) (layer "F.Cu") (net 5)))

